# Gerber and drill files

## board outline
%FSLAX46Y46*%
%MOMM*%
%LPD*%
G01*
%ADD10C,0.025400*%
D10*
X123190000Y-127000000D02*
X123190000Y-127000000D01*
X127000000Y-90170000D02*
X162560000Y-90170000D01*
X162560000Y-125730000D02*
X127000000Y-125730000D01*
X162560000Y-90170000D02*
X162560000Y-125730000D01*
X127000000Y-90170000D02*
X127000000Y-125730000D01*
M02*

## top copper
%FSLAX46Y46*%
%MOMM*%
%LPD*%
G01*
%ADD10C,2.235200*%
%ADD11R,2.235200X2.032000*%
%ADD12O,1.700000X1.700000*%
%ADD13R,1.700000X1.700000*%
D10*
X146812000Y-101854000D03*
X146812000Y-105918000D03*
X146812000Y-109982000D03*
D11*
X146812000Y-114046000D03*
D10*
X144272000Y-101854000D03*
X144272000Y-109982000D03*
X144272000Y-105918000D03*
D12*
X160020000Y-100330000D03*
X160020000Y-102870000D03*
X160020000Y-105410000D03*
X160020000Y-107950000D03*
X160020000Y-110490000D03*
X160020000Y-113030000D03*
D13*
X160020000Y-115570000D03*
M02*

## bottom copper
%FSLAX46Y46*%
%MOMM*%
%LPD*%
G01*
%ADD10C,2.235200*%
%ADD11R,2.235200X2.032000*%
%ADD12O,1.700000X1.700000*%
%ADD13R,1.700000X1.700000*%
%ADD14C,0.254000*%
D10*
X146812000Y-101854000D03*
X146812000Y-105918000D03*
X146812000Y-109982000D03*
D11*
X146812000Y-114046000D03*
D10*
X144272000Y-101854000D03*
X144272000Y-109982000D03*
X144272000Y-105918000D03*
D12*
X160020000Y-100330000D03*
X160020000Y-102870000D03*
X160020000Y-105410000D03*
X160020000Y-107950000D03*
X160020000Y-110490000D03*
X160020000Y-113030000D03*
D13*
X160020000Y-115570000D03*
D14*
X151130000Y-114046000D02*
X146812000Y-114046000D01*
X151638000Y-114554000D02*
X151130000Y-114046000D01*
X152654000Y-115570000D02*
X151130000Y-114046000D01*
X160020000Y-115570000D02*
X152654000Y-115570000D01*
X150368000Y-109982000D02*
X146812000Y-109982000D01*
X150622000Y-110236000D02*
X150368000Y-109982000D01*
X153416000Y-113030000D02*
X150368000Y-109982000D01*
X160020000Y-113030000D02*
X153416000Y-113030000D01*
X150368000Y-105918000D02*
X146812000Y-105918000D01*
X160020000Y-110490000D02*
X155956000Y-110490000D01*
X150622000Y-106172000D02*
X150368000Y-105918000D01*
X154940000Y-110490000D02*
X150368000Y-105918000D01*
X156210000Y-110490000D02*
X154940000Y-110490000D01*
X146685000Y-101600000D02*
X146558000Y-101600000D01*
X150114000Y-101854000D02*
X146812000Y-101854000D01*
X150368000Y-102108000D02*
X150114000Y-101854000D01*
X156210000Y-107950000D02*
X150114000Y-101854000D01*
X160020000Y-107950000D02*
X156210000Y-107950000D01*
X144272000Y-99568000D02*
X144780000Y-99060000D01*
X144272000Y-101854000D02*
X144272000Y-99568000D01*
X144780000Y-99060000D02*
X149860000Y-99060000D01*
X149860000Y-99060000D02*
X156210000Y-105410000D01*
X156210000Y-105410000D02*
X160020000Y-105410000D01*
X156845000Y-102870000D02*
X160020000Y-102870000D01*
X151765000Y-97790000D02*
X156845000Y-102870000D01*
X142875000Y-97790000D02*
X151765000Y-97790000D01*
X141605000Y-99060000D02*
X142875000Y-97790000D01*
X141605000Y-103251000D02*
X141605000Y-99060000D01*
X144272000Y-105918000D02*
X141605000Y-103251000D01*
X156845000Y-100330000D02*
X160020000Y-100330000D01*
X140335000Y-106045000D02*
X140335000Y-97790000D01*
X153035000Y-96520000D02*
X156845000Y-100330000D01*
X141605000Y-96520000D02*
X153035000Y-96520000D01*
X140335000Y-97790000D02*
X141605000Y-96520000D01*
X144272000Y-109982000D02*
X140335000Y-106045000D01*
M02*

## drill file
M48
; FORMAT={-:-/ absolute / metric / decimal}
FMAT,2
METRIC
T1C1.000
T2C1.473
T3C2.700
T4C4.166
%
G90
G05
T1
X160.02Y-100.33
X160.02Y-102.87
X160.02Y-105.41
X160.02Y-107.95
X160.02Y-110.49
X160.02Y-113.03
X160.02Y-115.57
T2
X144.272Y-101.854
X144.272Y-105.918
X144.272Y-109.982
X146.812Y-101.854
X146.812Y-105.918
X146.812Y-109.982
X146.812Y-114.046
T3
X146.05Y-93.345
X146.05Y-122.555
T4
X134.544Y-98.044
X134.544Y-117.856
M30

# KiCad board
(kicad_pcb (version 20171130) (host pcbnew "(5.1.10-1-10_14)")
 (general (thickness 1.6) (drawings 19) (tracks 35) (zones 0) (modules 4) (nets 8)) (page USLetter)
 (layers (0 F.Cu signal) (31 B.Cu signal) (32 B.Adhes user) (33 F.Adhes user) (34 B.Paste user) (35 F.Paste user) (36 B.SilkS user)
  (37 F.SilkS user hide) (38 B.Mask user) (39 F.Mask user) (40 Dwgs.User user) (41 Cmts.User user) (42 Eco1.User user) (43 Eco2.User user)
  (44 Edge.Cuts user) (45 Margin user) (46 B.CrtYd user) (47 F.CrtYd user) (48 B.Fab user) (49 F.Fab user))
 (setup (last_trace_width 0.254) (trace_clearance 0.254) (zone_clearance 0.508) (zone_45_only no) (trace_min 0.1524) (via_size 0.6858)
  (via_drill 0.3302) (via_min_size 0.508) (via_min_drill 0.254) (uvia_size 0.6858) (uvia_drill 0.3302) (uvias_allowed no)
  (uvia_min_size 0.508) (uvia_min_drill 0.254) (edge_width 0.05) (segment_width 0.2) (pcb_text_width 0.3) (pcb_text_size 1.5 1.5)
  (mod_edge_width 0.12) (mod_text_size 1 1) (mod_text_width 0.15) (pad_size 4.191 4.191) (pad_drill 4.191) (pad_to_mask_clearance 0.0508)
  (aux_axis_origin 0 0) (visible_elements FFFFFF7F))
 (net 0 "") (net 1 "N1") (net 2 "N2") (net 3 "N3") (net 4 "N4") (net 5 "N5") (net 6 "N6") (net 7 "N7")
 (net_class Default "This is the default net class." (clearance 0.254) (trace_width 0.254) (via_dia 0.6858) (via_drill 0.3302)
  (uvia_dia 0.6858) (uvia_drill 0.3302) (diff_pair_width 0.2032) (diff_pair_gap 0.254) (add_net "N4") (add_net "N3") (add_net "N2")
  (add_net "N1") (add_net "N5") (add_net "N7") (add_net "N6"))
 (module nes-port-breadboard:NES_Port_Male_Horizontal (layer F.Cu) (at 147.574 107.95)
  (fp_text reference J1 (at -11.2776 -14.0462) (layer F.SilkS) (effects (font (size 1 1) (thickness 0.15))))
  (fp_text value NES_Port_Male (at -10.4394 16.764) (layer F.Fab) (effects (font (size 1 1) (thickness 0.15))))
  (pad 4 thru_hole circle (at -0.762 -6.096) (size 2.2352 2.2352) (drill 1.4732) (layers *.Cu *.Mask) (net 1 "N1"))
  (pad 3 thru_hole circle (at -0.762 -2.032) (size 2.2352 2.2352) (drill 1.4732) (layers *.Cu *.Mask) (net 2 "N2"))
  (pad 2 thru_hole circle (at -0.762 2.032) (size 2.2352 2.2352) (drill 1.4732) (layers *.Cu *.Mask) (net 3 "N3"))
  (pad 1 thru_hole rect (at -0.762 6.096) (size 2.2352 2.032) (drill 1.4732) (layers *.Cu *.Mask) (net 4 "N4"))
  (pad 5 thru_hole circle (at -3.302 -6.096) (size 2.2352 2.2352) (drill 1.4732) (layers *.Cu *.Mask) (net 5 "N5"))
  (pad 7 thru_hole circle (at -3.302 2.032) (size 2.2352 2.2352) (drill 1.4732) (layers *.Cu *.Mask) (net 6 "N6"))
  (pad 6 thru_hole circle (at -3.302 -2.032) (size 2.2352 2.2352) (drill 1.4732) (layers *.Cu *.Mask) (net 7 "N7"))
  (pad "" np_thru_hole circle (at -13.0302 -9.906) (size 4.1656 4.1656) (drill 4.1656) (layers *.Cu *.Mask))
  (pad "" np_thru_hole circle (at -13.0302 9.906) (size 4.1656 4.1656) (drill 4.1656) (layers *.Cu *.Mask)))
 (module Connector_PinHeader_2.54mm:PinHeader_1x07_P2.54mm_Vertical (layer B.Cu) (at 160.02 115.57)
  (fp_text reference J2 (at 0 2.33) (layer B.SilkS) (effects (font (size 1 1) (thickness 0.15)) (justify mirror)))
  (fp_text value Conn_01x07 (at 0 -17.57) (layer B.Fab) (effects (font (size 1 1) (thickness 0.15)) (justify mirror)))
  (pad 7 thru_hole oval (at 0 -15.24) (size 1.7 1.7) (drill 1) (layers *.Cu *.Mask) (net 6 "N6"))
  (pad 6 thru_hole oval (at 0 -12.7) (size 1.7 1.7) (drill 1) (layers *.Cu *.Mask) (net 7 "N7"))
  (pad 5 thru_hole oval (at 0 -10.16) (size 1.7 1.7) (drill 1) (layers *.Cu *.Mask) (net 5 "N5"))
  (pad 4 thru_hole oval (at 0 -7.62) (size 1.7 1.7) (drill 1) (layers *.Cu *.Mask) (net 1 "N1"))
  (pad 3 thru_hole oval (at 0 -5.08) (size 1.7 1.7) (drill 1) (layers *.Cu *.Mask) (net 2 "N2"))
  (pad 2 thru_hole oval (at 0 -2.54) (size 1.7 1.7) (drill 1) (layers *.Cu *.Mask) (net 3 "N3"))
  (pad 1 thru_hole rect (at 0 0) (size 1.7 1.7) (drill 1) (layers *.Cu *.Mask) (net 4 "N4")))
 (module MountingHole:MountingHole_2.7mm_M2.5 (layer F.Cu) (at 146.05 122.555)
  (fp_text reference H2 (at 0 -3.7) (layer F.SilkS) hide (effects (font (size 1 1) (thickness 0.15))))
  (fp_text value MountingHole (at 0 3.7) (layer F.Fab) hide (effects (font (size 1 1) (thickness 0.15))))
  (pad 1 np_thru_hole circle (at 0 0) (size 2.7 2.7) (drill 2.7) (layers *.Cu *.Mask)))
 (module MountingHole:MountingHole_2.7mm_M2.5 (layer F.Cu) (at 146.05 93.345)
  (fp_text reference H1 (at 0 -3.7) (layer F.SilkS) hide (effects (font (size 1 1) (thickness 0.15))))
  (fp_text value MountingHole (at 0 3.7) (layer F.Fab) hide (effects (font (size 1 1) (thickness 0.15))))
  (pad 1 np_thru_hole circle (at 0 0) (size 2.7 2.7) (drill 2.7) (layers *.Cu *.Mask)))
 (gr_line (start 123.19 127) (end 123.19 127) (layer Edge.Cuts) (width 0.0254))
 (gr_line (start 127 90.17) (end 162.56 90.17) (layer Edge.Cuts) (width 0.0254))
 (gr_line (start 162.56 125.73) (end 127 125.73) (layer Edge.Cuts) (width 0.0254))
 (gr_line (start 162.56 90.17) (end 162.56 125.73) (layer Edge.Cuts) (width 0.0254))
 (gr_line (start 127 90.17) (end 127 125.73) (layer Edge.Cuts) (width 0.0254))
 (segment (start 151.13 114.046) (end 146.812 114.046) (width 0.254) (layer B.Cu) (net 4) (status 20))
 (segment (start 151.638 114.554) (end 151.13 114.046) (width 0.254) (layer B.Cu) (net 4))
 (segment (start 152.654 115.57) (end 151.13 114.046) (width 0.254) (layer B.Cu) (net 4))
 (segment (start 160.02 115.57) (end 152.654 115.57) (width 0.254) (layer B.Cu) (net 4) (status 10))
 (segment (start 150.368 109.982) (end 146.812 109.982) (width 0.254) (layer B.Cu) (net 3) (status 20))
 (segment (start 150.622 110.236) (end 150.368 109.982) (width 0.254) (layer B.Cu) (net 3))
 (segment (start 153.416 113.03) (end 150.368 109.982) (width 0.254) (layer B.Cu) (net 3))
 (segment (start 160.02 113.03) (end 153.416 113.03) (width 0.254) (layer B.Cu) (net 3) (status 10))
 (segment (start 150.368 105.918) (end 146.812 105.918) (width 0.254) (layer B.Cu) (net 2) (status 20))
 (segment (start 160.02 110.49) (end 155.956 110.49) (width 0.254) (layer B.Cu) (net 2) (status 10))
 (segment (start 150.622 106.172) (end 150.368 105.918) (width 0.254) (layer B.Cu) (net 2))
 (segment (start 154.94 110.49) (end 150.368 105.918) (width 0.254) (layer B.Cu) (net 2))
 (segment (start 156.21 110.49) (end 154.94 110.49) (width 0.254) (layer B.Cu) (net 2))
 (segment (start 146.685 101.6) (end 146.558 101.6) (width 0.254) (layer B.Cu) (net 1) (status 30))
 (segment (start 150.114 101.854) (end 146.812 101.854) (width 0.254) (layer B.Cu) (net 1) (status 20))
 (segment (start 150.368 102.108) (end 150.114 101.854) (width 0.254) (layer B.Cu) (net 1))
 (segment (start 156.21 107.95) (end 150.114 101.854) (width 0.254) (layer B.Cu) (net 1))
 (segment (start 160.02 107.95) (end 156.21 107.95) (width 0.254) (layer B.Cu) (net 1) (status 10))
 (segment (start 144.272 99.568) (end 144.78 99.06) (width 0.254) (layer B.Cu) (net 5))
 (segment (start 144.272 101.854) (end 144.272 99.568) (width 0.254) (layer B.Cu) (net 5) (status 10))
 (segment (start 144.78 99.06) (end 149.86 99.06) (width 0.254) (layer B.Cu) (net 5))
 (segment (start 149.86 99.06) (end 156.21 105.41) (width 0.254) (layer B.Cu) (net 5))
 (segment (start 156.21 105.41) (end 160.02 105.41) (width 0.254) (layer B.Cu) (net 5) (status 20))
 (segment (start 156.845 102.87) (end 160.02 102.87) (width 0.254) (layer B.Cu) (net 7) (status 20))
 (segment (start 151.765 97.79) (end 156.845 102.87) (width 0.254) (layer B.Cu) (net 7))
 (segment (start 142.875 97.79) (end 151.765 97.79) (width 0.254) (layer B.Cu) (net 7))
 (segment (start 141.605 99.06) (end 142.875 97.79) (width 0.254) (layer B.Cu) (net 7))
 (segment (start 141.605 103.251) (end 141.605 99.06) (width 0.254) (layer B.Cu) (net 7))
 (segment (start 144.272 105.918) (end 141.605 103.251) (width 0.254) (layer B.Cu) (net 7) (status 10))
 (segment (start 156.845 100.33) (end 160.02 100.33) (width 0.254) (layer B.Cu) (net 6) (status 20))
 (segment (start 140.335 106.045) (end 140.335 97.79) (width 0.254) (layer B.Cu) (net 6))
 (segment (start 153.035 96.52) (end 156.845 100.33) (width 0.254) (layer B.Cu) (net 6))
 (segment (start 141.605 96.52) (end 153.035 96.52) (width 0.254) (layer B.Cu) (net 6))
 (segment (start 140.335 97.79) (end 141.605 96.52) (width 0.254) (layer B.Cu) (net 6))
 (segment (start 144.272 109.982) (end 140.335 106.045) (width 0.254) (layer B.Cu) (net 6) (status 10)))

